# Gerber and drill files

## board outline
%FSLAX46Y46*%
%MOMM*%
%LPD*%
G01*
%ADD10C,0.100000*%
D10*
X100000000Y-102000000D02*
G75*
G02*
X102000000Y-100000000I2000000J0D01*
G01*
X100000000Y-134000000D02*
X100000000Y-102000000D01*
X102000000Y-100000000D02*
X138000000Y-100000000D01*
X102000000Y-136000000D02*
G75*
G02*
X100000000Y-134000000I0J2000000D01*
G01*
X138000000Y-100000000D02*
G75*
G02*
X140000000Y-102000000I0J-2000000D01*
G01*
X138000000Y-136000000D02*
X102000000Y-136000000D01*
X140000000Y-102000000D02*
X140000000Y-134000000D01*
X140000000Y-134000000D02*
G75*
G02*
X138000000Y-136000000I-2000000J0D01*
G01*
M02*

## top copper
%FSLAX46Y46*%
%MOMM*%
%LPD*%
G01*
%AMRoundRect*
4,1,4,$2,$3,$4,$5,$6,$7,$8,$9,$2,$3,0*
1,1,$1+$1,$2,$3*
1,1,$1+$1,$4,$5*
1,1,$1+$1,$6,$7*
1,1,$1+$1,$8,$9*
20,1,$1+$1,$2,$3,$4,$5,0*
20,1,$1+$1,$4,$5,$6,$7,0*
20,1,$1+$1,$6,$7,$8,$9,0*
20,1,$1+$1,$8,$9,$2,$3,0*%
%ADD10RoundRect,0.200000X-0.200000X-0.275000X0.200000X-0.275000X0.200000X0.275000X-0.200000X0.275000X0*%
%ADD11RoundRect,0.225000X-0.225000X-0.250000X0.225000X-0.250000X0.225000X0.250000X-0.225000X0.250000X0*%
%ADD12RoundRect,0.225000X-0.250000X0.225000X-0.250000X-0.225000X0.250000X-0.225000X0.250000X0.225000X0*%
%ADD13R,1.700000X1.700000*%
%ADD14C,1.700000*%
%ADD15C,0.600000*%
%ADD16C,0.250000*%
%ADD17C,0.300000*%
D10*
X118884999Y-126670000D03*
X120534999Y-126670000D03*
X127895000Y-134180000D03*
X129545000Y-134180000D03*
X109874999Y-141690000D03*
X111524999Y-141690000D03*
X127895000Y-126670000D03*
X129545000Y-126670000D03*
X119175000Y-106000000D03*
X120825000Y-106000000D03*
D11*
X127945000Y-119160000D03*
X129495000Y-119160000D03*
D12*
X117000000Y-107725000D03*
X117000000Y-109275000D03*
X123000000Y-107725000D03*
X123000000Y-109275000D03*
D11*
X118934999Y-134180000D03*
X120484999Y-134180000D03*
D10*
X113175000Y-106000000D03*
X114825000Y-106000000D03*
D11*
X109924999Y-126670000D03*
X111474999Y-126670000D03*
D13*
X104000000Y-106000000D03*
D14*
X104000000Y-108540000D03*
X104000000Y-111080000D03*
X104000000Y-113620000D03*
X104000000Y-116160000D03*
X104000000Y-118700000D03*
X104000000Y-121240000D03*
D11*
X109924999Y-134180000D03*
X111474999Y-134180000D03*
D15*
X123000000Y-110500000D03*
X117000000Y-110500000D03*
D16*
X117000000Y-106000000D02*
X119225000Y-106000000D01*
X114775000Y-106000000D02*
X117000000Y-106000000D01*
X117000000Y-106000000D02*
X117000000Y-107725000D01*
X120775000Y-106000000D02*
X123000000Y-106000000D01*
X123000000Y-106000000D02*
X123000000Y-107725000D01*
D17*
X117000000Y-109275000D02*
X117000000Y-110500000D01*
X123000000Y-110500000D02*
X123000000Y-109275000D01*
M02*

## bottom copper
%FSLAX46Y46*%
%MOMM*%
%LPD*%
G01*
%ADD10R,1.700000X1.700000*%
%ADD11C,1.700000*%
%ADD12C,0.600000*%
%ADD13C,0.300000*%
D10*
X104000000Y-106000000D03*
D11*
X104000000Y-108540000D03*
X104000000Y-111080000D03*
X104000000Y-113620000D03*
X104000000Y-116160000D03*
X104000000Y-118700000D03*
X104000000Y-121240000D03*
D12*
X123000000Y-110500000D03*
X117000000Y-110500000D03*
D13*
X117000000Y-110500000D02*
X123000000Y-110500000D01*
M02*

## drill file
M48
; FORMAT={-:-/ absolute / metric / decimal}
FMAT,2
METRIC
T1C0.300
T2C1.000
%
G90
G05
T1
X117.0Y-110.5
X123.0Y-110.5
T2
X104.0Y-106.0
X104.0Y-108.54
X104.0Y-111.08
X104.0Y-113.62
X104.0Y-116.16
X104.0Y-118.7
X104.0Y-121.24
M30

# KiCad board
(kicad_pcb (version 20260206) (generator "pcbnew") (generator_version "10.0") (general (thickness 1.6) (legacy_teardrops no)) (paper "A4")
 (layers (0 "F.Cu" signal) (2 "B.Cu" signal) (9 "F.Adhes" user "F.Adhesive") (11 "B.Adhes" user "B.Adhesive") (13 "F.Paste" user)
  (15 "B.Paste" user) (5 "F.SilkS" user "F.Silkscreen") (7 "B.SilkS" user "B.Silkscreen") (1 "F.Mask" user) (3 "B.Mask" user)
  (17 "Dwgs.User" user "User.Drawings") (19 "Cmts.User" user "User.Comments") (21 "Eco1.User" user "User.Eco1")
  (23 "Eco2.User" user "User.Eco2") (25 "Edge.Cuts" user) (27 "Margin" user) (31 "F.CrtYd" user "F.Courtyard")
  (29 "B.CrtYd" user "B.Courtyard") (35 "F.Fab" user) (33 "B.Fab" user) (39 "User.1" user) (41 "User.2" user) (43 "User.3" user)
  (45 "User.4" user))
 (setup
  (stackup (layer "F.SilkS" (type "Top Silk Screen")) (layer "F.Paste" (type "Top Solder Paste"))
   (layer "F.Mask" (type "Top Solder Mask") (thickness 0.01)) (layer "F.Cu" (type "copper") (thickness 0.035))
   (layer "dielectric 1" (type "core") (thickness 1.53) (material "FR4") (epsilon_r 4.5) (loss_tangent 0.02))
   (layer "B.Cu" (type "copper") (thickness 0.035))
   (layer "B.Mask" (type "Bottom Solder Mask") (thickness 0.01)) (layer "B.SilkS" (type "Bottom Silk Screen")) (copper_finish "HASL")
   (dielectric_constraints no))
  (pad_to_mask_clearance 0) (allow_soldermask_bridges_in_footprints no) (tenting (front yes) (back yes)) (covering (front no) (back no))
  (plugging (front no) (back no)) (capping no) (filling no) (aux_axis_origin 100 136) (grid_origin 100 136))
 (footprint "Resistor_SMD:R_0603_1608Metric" (layer "F.Cu") (at 119.709999 126.67)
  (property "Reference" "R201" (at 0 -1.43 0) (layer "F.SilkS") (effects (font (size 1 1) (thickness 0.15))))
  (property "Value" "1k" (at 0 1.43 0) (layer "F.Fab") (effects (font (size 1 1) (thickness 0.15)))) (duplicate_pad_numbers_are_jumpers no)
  (pad "1" smd roundrect (at -0.825 0) (size 0.8 0.95) (layers "F.Cu" "F.Mask" "F.Paste") (roundrect_rratio 0.25) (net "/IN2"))
  (pad "2" smd roundrect (at 0.825 0) (size 0.8 0.95) (layers "F.Cu" "F.Mask" "F.Paste") (roundrect_rratio 0.25) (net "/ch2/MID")))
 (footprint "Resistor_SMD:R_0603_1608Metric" (layer "F.Cu") (at 128.72 134.18)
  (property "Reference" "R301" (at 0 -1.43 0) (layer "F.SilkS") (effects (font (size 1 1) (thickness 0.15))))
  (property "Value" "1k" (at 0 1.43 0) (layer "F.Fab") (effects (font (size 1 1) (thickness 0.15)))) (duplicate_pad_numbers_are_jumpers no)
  (pad "1" smd roundrect (at -0.825 0) (size 0.8 0.95) (layers "F.Cu" "F.Mask" "F.Paste") (roundrect_rratio 0.25) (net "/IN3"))
  (pad "2" smd roundrect (at 0.825 0) (size 0.8 0.95) (layers "F.Cu" "F.Mask" "F.Paste") (roundrect_rratio 0.25) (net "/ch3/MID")))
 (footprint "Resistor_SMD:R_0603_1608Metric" (layer "F.Cu") (at 110.699999 141.69)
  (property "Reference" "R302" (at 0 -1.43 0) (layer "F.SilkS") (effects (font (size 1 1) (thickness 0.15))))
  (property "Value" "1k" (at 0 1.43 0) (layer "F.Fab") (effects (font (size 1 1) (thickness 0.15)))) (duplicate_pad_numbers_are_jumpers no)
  (pad "1" smd roundrect (at -0.825 0) (size 0.8 0.95) (layers "F.Cu" "F.Mask" "F.Paste") (roundrect_rratio 0.25) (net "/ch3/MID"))
  (pad "2" smd roundrect (at 0.825 0) (size 0.8 0.95) (layers "F.Cu" "F.Mask" "F.Paste") (roundrect_rratio 0.25) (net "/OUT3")))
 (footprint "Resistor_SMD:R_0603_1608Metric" (layer "F.Cu") (at 128.72 126.67)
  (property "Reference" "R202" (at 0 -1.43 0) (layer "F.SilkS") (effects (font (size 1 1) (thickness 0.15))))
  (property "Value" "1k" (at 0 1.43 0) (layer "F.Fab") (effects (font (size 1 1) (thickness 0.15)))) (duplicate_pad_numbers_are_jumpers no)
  (pad "1" smd roundrect (at -0.825 0) (size 0.8 0.95) (layers "F.Cu" "F.Mask" "F.Paste") (roundrect_rratio 0.25) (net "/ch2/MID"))
  (pad "2" smd roundrect (at 0.825 0) (size 0.8 0.95) (layers "F.Cu" "F.Mask" "F.Paste") (roundrect_rratio 0.25) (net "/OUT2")))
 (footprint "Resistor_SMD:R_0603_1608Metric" (layer "F.Cu") (at 120 106)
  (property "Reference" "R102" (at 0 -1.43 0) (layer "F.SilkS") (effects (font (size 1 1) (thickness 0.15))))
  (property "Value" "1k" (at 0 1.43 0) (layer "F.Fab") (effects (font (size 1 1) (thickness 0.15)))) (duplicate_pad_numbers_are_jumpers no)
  (pad "1" smd roundrect (at -0.825 0) (size 0.8 0.95) (layers "F.Cu" "F.Mask" "F.Paste") (roundrect_rratio 0.25) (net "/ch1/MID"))
  (pad "2" smd roundrect (at 0.825 0) (size 0.8 0.95) (layers "F.Cu" "F.Mask" "F.Paste") (roundrect_rratio 0.25) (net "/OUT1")))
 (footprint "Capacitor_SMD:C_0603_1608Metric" (layer "F.Cu") (at 128.72 119.16)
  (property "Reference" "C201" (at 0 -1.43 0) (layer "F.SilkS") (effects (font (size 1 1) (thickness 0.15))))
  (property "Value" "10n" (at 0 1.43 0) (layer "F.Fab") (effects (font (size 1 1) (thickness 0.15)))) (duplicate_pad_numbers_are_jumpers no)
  (pad "1" smd roundrect (at -0.775 0) (size 0.9 0.95) (layers "F.Cu" "F.Mask" "F.Paste") (roundrect_rratio 0.25) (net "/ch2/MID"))
  (pad "2" smd roundrect (at 0.775 0) (size 0.9 0.95) (layers "F.Cu" "F.Mask" "F.Paste") (roundrect_rratio 0.25) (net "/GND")))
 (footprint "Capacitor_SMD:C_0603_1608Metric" (layer "F.Cu") (at 117 108.5 -90)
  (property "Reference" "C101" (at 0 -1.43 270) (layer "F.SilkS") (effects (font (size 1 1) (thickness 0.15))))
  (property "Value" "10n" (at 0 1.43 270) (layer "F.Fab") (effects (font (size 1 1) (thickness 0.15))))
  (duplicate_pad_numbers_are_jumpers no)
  (pad "1" smd roundrect (at -0.775 0 270) (size 0.9 0.95) (layers "F.Cu" "F.Mask" "F.Paste") (roundrect_rratio 0.25) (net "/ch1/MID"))
  (pad "2" smd roundrect (at 0.775 0 270) (size 0.9 0.95) (layers "F.Cu" "F.Mask" "F.Paste") (roundrect_rratio 0.25) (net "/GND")))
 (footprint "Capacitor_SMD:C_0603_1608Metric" (layer "F.Cu") (at 123 108.5 -90)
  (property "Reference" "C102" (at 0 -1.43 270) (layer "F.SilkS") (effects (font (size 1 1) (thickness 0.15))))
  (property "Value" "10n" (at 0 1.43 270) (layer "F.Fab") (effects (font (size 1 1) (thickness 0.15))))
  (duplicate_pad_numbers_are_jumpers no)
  (pad "1" smd roundrect (at -0.775 0 270) (size 0.9 0.95) (layers "F.Cu" "F.Mask" "F.Paste") (roundrect_rratio 0.25) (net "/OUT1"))
  (pad "2" smd roundrect (at 0.775 0 270) (size 0.9 0.95) (layers "F.Cu" "F.Mask" "F.Paste") (roundrect_rratio 0.25) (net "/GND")))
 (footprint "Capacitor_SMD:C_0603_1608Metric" (layer "F.Cu") (at 119.709999 134.18)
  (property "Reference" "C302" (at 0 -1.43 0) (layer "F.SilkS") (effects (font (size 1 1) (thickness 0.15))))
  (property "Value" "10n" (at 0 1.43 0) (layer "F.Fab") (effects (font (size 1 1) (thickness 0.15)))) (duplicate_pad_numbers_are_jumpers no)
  (pad "1" smd roundrect (at -0.775 0) (size 0.9 0.95) (layers "F.Cu" "F.Mask" "F.Paste") (roundrect_rratio 0.25) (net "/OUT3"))
  (pad "2" smd roundrect (at 0.775 0) (size 0.9 0.95) (layers "F.Cu" "F.Mask" "F.Paste") (roundrect_rratio 0.25) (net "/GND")))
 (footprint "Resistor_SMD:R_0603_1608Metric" (layer "F.Cu") (at 114 106)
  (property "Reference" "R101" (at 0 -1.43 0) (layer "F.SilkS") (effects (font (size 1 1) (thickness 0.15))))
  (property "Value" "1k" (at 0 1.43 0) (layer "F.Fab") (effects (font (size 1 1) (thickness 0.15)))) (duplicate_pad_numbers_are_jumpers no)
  (pad "1" smd roundrect (at -0.825 0) (size 0.8 0.95) (layers "F.Cu" "F.Mask" "F.Paste") (roundrect_rratio 0.25) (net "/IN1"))
  (pad "2" smd roundrect (at 0.825 0) (size 0.8 0.95) (layers "F.Cu" "F.Mask" "F.Paste") (roundrect_rratio 0.25) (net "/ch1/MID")))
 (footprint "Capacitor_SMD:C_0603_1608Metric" (layer "F.Cu") (at 110.699999 126.67)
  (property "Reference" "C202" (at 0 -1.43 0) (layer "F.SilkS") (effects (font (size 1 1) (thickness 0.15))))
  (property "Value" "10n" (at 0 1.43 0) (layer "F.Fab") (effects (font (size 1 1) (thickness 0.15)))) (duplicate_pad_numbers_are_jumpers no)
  (pad "1" smd roundrect (at -0.775 0) (size 0.9 0.95) (layers "F.Cu" "F.Mask" "F.Paste") (roundrect_rratio 0.25) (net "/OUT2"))
  (pad "2" smd roundrect (at 0.775 0) (size 0.9 0.95) (layers "F.Cu" "F.Mask" "F.Paste") (roundrect_rratio 0.25) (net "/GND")))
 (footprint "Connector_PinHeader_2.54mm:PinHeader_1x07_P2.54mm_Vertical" (layer "F.Cu") (at 104 106)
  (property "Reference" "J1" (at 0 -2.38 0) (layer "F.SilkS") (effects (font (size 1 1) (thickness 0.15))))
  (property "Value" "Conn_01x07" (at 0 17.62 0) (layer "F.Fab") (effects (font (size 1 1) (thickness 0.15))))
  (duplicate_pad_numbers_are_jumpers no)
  (pad "1" thru_hole rect (at 0 0) (size 1.7 1.7) (drill 1) (layers "*.Cu" "*.Mask") (remove_unused_layers no) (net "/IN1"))
  (pad "2" thru_hole circle (at 0 2.54) (size 1.7 1.7) (drill 1) (layers "*.Cu" "*.Mask") (remove_unused_layers no) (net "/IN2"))
  (pad "3" thru_hole circle (at 0 5.08) (size 1.7 1.7) (drill 1) (layers "*.Cu" "*.Mask") (remove_unused_layers no) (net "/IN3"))
  (pad "4" thru_hole circle (at 0 7.62) (size 1.7 1.7) (drill 1) (layers "*.Cu" "*.Mask") (remove_unused_layers no) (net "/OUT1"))
  (pad "5" thru_hole circle (at 0 10.16) (size 1.7 1.7) (drill 1) (layers "*.Cu" "*.Mask") (remove_unused_layers no) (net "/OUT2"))
  (pad "6" thru_hole circle (at 0 12.7) (size 1.7 1.7) (drill 1) (layers "*.Cu" "*.Mask") (remove_unused_layers no) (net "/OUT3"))
  (pad "7" thru_hole circle (at 0 15.24) (size 1.7 1.7) (drill 1) (layers "*.Cu" "*.Mask") (remove_unused_layers no) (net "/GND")))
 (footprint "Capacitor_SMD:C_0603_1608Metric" (layer "F.Cu") (at 110.699999 134.18)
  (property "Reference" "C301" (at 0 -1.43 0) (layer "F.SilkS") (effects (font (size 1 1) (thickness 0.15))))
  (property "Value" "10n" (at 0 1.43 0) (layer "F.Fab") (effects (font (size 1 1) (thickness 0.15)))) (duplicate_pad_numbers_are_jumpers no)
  (pad "1" smd roundrect (at -0.775 0) (size 0.9 0.95) (layers "F.Cu" "F.Mask" "F.Paste") (roundrect_rratio 0.25) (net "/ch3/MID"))
  (pad "2" smd roundrect (at 0.775 0) (size 0.9 0.95) (layers "F.Cu" "F.Mask" "F.Paste") (roundrect_rratio 0.25) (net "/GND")))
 (gr_arc (start 100 102) (mid 100.585786 100.585786) (end 102 100) (stroke (width 0.1) (type default)) (layer "Edge.Cuts"))
 (gr_line (start 100 134) (end 100 102) (stroke (width 0.1) (type default)) (layer "Edge.Cuts"))
 (gr_line (start 102 100) (end 138 100) (stroke (width 0.1) (type default)) (layer "Edge.Cuts"))
 (gr_arc (start 102 136) (mid 100.585786 135.414213) (end 100 134) (stroke (width 0.1) (type default)) (layer "Edge.Cuts"))
 (gr_arc (start 138 100) (mid 139.414213 100.585786) (end 140 102) (stroke (width 0.1) (type default)) (layer "Edge.Cuts"))
 (gr_line (start 138 136) (end 102 136) (stroke (width 0.1) (type default)) (layer "Edge.Cuts"))
 (gr_line (start 140 102) (end 140 134) (stroke (width 0.1) (type default)) (layer "Edge.Cuts"))
 (gr_arc (start 140 134) (mid 139.414213 135.414213) (end 138 136) (stroke (width 0.1) (type default)) (layer "Edge.Cuts"))
 (segment (start 117 106) (end 119.225 106) (width 0.25) (layer "F.Cu") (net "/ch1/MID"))
 (segment (start 114.775 106) (end 117 106) (width 0.25) (layer "F.Cu") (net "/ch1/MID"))
 (segment (start 117 106) (end 117 107.725) (width 0.25) (layer "F.Cu") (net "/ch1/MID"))
 (segment (start 120.775 106) (end 123 106) (width 0.25) (layer "F.Cu") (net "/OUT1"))
 (segment (start 123 106) (end 123 107.725) (width 0.25) (layer "F.Cu") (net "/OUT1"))
 (segment (start 117 109.275) (end 117 110.5) (width 0.3) (layer "F.Cu") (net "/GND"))
 (segment (start 123 110.5) (end 123 109.275) (width 0.3) (layer "F.Cu") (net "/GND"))
 (via (at 123 110.5) (size 0.6) (drill 0.3) (layers "F.Cu" "B.Cu") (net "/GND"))
 (via (at 117 110.5) (size 0.6) (drill 0.3) (layers "F.Cu" "B.Cu") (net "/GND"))
 (segment (start 117 110.5) (end 123 110.5) (width 0.3) (layer "B.Cu") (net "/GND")))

